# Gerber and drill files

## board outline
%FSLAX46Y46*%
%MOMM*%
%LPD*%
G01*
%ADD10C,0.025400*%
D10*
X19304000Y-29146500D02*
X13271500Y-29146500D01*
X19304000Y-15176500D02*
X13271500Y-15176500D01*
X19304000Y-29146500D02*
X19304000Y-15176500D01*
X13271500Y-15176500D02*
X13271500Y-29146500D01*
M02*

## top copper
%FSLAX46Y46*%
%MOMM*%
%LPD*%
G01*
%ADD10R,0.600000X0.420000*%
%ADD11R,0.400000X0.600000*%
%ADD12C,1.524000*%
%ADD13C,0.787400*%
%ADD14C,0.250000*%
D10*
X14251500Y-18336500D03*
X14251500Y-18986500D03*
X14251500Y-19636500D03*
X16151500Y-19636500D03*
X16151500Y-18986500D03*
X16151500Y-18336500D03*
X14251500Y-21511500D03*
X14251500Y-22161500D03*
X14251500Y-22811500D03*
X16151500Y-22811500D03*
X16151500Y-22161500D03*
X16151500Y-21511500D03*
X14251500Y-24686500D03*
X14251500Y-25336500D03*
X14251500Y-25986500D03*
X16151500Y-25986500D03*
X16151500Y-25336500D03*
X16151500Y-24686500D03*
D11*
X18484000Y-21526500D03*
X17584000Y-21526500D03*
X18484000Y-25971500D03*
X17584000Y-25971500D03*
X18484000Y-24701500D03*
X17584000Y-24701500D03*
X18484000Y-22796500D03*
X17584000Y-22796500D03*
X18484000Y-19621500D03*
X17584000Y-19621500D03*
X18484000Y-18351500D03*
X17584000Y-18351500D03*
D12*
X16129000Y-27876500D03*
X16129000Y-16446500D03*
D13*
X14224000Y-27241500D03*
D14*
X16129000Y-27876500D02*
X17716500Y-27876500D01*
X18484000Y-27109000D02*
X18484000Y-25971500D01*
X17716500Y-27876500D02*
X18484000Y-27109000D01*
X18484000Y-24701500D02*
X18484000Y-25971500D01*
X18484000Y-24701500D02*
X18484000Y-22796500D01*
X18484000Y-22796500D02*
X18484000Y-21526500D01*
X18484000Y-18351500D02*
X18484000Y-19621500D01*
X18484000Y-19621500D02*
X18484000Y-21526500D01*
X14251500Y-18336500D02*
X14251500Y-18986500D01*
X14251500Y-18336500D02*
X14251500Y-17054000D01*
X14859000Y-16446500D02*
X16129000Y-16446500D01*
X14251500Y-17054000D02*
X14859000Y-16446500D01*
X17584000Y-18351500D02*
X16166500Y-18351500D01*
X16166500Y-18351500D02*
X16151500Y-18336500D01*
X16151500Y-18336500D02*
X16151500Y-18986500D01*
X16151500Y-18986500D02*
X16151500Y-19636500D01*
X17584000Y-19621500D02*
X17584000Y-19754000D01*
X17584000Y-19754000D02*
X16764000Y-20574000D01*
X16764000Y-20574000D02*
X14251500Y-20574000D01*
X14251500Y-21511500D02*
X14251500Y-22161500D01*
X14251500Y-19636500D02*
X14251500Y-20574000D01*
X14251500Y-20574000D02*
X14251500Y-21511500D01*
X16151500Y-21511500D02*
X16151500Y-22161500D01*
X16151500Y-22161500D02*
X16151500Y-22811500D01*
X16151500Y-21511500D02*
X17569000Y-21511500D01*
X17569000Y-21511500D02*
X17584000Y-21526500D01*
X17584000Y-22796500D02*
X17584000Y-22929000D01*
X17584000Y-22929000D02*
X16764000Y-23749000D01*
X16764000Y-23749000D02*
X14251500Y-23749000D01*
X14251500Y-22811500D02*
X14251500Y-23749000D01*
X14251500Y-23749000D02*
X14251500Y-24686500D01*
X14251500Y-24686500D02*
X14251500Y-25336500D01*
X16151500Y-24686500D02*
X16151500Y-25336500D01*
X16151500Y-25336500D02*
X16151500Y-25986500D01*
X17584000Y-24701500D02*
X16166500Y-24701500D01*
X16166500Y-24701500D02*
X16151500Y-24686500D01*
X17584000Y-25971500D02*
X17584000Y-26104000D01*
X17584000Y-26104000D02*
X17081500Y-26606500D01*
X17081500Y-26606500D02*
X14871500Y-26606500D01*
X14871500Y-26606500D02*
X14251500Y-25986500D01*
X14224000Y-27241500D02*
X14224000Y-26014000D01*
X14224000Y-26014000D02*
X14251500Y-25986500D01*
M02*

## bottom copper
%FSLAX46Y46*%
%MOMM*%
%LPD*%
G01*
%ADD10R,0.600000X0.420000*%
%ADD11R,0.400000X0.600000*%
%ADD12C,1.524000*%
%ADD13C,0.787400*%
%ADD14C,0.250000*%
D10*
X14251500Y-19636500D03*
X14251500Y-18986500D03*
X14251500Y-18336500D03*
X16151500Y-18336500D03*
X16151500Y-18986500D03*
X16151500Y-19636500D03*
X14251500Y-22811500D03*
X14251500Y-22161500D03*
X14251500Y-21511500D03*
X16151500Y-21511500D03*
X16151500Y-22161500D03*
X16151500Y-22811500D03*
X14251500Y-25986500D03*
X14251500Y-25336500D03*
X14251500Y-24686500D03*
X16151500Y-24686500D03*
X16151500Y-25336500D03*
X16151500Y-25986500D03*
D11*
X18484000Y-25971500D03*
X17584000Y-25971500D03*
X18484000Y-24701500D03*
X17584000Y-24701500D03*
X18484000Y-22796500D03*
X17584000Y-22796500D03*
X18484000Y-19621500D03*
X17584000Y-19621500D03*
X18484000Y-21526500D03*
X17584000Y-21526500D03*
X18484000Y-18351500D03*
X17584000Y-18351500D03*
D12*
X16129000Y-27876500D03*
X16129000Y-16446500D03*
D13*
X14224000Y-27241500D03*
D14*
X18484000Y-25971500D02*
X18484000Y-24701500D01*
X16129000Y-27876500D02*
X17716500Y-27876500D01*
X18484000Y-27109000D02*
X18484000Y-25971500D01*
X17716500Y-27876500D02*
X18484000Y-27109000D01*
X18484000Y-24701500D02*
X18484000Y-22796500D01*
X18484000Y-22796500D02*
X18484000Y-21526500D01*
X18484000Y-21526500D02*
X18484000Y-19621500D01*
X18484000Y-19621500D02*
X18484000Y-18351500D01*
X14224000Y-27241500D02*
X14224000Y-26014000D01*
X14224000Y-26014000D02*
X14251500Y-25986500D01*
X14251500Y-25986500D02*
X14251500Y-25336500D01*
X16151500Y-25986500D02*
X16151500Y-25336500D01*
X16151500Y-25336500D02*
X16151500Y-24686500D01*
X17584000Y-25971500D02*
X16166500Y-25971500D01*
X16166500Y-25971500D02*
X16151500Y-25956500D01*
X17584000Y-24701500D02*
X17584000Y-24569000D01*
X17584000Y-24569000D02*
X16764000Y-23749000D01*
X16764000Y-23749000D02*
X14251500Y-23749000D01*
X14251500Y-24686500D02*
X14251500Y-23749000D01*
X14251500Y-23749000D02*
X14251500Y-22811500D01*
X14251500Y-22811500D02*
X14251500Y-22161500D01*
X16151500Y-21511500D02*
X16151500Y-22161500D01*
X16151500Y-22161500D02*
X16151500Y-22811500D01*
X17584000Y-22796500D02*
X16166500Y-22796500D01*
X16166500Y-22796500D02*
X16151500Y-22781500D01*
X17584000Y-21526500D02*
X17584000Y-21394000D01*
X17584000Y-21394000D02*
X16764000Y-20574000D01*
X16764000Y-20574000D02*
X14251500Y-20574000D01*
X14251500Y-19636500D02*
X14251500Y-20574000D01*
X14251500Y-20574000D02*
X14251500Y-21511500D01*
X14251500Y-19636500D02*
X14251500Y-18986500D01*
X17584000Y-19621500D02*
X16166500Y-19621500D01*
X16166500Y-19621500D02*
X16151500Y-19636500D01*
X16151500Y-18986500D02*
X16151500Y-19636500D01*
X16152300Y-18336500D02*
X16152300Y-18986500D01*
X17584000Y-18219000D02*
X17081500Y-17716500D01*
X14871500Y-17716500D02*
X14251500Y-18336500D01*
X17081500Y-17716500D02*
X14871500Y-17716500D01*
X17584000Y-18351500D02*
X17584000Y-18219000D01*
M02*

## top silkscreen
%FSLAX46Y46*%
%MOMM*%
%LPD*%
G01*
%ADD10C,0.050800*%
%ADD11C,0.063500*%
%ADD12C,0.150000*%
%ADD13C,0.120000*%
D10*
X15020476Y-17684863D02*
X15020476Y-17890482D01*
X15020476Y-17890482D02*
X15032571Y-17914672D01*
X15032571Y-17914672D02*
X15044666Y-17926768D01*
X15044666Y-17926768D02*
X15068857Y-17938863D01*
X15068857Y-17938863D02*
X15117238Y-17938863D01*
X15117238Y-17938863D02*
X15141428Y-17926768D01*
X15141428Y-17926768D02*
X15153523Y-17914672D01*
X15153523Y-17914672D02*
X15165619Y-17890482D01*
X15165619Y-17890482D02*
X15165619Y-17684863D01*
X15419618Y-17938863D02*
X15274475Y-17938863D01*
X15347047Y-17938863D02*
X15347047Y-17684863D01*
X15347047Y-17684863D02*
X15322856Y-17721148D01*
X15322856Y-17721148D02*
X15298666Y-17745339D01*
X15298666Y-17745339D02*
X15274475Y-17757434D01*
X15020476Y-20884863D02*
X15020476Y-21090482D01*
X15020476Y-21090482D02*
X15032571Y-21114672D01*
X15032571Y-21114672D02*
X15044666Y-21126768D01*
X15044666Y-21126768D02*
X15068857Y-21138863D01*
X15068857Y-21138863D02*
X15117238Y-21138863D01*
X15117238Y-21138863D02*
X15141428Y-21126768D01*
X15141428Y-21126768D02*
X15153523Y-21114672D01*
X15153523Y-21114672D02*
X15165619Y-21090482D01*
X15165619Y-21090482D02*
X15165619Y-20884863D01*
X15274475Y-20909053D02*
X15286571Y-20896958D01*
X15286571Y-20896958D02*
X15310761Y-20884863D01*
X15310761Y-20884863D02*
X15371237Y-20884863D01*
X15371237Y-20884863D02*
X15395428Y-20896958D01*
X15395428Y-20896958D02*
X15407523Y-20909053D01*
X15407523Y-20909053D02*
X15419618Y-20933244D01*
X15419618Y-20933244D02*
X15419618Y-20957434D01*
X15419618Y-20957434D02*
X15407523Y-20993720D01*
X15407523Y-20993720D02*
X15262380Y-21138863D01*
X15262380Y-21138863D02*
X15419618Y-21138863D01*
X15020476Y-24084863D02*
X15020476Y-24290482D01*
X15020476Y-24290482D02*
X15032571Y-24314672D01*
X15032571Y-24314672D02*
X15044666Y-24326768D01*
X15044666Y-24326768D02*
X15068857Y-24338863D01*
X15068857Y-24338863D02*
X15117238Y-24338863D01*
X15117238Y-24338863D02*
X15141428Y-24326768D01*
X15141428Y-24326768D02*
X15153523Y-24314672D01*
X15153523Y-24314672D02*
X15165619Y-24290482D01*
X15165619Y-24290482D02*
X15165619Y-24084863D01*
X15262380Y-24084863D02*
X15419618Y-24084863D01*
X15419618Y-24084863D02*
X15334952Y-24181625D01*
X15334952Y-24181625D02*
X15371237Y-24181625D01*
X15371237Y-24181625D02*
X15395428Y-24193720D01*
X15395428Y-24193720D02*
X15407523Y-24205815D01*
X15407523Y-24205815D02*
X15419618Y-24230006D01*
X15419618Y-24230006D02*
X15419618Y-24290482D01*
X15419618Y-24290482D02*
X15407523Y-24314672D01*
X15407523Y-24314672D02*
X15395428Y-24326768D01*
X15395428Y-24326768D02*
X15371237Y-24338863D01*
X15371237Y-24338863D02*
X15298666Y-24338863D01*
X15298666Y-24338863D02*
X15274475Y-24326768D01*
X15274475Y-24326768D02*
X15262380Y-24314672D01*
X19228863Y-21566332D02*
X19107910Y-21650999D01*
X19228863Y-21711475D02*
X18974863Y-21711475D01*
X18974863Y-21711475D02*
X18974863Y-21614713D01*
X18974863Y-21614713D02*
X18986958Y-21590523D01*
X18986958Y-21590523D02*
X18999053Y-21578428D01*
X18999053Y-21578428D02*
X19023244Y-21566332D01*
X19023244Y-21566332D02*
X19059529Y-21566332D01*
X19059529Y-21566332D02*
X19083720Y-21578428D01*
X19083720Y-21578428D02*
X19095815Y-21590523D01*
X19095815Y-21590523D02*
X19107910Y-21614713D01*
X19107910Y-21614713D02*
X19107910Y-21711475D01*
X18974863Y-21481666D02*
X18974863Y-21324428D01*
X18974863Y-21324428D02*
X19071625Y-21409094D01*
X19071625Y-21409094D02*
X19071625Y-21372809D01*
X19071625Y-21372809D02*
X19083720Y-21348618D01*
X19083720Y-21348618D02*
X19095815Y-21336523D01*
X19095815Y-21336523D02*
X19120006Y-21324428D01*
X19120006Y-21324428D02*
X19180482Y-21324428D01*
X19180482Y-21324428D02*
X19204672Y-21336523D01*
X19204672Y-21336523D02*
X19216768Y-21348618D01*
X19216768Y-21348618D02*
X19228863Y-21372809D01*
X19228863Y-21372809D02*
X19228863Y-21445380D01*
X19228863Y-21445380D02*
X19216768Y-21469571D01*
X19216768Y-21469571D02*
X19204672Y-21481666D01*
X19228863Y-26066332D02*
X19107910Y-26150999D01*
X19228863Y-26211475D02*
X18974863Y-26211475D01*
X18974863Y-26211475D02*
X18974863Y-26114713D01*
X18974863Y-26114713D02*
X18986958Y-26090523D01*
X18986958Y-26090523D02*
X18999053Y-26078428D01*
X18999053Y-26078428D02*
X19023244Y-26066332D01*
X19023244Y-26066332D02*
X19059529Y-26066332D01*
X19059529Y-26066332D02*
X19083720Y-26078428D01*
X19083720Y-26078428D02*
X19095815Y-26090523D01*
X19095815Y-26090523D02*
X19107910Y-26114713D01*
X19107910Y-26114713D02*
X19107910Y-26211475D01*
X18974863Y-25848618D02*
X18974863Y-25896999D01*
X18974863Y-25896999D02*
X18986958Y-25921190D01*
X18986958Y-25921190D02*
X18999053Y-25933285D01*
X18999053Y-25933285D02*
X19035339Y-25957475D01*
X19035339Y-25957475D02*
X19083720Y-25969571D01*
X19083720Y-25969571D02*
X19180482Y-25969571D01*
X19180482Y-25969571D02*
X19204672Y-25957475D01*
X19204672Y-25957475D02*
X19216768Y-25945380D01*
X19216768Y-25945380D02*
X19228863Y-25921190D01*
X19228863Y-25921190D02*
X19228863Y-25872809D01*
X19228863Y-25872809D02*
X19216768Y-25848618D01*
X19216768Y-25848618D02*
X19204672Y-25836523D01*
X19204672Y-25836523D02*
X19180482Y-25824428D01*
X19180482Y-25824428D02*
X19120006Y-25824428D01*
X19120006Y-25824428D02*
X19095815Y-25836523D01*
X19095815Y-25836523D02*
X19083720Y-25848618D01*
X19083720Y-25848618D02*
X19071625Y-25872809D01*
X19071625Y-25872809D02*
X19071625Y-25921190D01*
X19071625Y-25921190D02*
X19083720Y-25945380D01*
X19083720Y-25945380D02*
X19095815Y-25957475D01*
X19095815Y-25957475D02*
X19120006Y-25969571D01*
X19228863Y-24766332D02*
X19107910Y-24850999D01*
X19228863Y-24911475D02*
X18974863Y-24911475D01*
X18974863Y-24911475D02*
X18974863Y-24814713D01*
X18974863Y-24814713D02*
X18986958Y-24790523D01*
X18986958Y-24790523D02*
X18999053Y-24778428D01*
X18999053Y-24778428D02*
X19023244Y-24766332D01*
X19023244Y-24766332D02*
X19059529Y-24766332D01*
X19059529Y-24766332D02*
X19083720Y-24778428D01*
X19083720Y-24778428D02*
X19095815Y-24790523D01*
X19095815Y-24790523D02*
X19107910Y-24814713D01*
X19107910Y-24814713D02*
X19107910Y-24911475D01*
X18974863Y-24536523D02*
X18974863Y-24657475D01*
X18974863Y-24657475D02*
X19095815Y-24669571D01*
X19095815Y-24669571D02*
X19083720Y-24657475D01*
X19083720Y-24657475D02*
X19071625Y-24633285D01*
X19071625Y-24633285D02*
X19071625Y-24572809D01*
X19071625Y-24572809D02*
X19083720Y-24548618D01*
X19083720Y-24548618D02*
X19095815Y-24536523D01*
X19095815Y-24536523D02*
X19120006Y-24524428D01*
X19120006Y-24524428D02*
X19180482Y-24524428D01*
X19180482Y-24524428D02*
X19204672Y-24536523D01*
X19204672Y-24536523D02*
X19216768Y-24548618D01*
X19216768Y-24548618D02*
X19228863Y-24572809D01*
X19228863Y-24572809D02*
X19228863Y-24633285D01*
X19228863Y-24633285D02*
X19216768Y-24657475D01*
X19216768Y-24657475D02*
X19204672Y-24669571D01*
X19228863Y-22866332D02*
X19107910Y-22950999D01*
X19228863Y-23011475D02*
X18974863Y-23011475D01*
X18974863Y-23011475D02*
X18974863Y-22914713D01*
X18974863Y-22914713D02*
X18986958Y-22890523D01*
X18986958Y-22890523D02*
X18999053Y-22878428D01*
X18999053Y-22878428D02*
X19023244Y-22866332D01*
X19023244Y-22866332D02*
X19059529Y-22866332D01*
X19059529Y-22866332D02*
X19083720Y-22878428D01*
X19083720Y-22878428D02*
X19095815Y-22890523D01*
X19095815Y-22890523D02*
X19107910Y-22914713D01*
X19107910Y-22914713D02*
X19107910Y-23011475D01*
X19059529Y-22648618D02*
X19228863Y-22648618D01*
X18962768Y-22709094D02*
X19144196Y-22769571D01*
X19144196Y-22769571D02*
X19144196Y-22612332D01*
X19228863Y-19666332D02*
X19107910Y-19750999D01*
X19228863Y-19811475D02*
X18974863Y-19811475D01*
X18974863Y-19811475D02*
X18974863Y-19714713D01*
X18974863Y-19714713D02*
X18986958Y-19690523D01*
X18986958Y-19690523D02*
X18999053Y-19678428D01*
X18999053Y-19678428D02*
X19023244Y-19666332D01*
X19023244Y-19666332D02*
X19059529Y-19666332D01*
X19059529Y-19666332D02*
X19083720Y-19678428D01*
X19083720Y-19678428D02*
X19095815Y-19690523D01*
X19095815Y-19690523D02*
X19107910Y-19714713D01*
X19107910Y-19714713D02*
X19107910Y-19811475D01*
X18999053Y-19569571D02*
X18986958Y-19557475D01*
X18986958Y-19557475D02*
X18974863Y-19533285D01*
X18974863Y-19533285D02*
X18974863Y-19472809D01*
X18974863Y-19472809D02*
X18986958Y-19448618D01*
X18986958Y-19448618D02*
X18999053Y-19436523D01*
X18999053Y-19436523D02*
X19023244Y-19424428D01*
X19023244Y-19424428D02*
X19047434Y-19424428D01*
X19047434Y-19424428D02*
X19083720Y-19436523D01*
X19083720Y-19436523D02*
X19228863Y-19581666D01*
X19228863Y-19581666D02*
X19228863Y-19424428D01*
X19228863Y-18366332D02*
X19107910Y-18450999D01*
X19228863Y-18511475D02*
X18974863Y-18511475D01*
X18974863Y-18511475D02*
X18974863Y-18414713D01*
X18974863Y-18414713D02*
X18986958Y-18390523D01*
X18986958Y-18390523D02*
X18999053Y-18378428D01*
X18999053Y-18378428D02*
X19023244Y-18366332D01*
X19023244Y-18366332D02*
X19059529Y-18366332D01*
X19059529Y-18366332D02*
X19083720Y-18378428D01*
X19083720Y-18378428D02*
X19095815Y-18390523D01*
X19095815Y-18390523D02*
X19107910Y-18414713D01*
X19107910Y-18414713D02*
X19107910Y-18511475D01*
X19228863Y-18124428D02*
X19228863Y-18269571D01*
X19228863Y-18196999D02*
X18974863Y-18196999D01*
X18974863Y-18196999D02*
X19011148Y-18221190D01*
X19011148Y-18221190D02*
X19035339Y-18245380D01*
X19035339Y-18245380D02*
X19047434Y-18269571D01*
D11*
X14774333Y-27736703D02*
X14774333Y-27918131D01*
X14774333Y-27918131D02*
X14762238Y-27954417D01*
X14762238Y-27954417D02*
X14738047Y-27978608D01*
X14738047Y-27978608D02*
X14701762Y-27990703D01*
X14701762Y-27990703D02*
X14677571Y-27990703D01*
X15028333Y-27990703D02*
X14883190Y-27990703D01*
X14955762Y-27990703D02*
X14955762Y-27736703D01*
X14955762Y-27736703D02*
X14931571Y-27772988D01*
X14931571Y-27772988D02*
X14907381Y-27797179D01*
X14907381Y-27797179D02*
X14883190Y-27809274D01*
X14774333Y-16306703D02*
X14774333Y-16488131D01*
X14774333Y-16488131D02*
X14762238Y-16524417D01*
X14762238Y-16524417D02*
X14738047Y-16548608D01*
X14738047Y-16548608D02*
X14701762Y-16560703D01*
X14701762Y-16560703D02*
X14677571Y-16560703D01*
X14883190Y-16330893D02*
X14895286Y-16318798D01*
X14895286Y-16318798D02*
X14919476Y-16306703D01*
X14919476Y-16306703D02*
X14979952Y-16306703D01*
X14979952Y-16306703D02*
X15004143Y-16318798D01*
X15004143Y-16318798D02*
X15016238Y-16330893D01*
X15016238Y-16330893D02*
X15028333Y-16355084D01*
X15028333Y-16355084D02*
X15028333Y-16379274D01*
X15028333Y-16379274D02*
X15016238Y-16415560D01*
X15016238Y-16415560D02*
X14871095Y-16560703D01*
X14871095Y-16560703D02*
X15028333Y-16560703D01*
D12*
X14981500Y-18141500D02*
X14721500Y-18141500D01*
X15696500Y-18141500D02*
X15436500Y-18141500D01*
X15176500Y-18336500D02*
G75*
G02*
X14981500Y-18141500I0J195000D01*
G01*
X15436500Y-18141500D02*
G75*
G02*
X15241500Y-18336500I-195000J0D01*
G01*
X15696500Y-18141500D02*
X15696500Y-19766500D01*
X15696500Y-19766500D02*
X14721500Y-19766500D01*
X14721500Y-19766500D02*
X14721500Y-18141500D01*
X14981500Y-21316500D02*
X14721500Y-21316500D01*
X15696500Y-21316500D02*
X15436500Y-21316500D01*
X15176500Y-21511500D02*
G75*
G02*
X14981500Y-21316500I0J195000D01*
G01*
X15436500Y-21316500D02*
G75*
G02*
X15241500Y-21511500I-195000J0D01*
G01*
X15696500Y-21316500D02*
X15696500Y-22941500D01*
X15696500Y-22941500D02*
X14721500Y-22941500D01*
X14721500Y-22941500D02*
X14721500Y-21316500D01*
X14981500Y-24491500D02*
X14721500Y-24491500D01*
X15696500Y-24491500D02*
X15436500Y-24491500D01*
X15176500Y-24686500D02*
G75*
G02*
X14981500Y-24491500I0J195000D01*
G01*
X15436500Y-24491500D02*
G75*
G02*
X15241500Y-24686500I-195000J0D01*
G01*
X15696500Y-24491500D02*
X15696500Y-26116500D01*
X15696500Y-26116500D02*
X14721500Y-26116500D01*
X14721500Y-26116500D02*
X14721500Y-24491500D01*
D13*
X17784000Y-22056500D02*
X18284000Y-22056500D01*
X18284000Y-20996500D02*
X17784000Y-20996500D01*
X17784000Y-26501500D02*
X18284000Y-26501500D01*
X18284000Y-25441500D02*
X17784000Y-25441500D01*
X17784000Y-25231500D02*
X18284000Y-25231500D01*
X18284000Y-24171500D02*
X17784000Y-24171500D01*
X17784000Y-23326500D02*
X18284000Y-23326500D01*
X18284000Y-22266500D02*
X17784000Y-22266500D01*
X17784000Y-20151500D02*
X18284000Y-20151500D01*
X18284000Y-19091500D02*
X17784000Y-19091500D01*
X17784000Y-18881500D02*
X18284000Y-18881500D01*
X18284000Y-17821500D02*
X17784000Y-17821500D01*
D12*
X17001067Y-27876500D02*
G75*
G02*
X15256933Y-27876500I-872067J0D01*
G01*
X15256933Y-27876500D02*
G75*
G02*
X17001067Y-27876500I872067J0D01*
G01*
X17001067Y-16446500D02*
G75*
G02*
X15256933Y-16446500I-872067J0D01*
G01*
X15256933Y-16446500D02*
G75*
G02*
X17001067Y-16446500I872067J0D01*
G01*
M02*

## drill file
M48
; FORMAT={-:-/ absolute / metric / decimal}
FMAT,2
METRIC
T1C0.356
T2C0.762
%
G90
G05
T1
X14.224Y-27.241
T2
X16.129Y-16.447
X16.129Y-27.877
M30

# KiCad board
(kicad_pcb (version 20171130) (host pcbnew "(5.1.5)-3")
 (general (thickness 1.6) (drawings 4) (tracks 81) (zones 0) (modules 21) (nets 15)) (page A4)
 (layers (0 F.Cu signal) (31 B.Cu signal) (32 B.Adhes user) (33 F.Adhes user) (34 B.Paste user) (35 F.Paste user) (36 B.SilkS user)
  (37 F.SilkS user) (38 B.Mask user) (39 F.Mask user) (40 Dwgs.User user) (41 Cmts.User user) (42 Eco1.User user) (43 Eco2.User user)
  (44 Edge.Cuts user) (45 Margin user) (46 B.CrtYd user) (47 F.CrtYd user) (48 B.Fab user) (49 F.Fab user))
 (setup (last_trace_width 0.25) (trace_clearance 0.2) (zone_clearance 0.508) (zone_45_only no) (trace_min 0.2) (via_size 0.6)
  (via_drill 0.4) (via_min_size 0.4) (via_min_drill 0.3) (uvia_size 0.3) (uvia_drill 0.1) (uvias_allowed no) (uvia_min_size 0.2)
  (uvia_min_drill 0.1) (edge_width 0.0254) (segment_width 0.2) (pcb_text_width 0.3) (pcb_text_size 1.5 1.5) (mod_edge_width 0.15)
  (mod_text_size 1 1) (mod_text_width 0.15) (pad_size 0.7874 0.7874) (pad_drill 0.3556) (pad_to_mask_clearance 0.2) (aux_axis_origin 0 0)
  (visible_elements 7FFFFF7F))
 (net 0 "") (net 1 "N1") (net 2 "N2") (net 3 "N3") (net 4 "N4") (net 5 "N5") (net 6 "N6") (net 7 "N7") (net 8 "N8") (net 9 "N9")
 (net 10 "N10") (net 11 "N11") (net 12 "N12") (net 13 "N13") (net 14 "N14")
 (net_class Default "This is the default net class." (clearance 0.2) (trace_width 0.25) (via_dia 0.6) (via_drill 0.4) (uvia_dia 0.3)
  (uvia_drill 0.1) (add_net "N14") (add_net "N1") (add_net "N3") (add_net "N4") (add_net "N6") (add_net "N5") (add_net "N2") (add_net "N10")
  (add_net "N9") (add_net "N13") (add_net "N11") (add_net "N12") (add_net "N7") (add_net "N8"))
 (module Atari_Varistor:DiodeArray (layer F.Cu) (at 15.1765 18.9865 270)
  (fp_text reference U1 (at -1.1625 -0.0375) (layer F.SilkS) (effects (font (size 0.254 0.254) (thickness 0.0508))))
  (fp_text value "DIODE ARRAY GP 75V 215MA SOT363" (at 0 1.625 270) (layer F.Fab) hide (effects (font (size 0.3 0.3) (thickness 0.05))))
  (fp_line (start -0.845 0.195) (end -0.845 0.455) (layer F.SilkS) (width 0.15))
  (fp_line (start -0.845 -0.52) (end -0.845 -0.26) (layer F.SilkS) (width 0.15))
  (fp_arc (start -0.845 0) (end -0.65 0) (angle 90) (layer F.SilkS) (width 0.15))
  (fp_arc (start -0.845 -0.065) (end -0.845 -0.26) (angle 90) (layer F.SilkS) (width 0.15))
  (fp_line (start -0.845 -0.52) (end 0.78 -0.52) (layer F.SilkS) (width 0.15))
  (fp_line (start 0.78 -0.52) (end 0.78 0.455) (layer F.SilkS) (width 0.15))
  (fp_line (start 0.78 0.455) (end -0.845 0.455) (layer F.SilkS) (width 0.15))
  (pad 1 smd rect (at -0.65 0.925 270) (size 0.42 0.6) (layers F.Cu F.Paste F.Mask) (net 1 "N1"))
  (pad 2 smd rect (at 0 0.925 270) (size 0.42 0.6) (layers F.Cu F.Paste F.Mask) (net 1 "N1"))
  (pad 3 smd rect (at 0.65 0.925 270) (size 0.42 0.6) (layers F.Cu F.Paste F.Mask) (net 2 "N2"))
  (pad 4 smd rect (at 0.65 -0.975 270) (size 0.42 0.6) (layers F.Cu F.Paste F.Mask) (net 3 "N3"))
  (pad 5 smd rect (at 0 -0.975 270) (size 0.42 0.6) (layers F.Cu F.Paste F.Mask) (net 3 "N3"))
  (pad 6 smd rect (at -0.65 -0.975 270) (size 0.42 0.6) (layers F.Cu F.Paste F.Mask) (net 3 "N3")))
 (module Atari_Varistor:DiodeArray (layer B.Cu) (at 15.1765 18.9865 90)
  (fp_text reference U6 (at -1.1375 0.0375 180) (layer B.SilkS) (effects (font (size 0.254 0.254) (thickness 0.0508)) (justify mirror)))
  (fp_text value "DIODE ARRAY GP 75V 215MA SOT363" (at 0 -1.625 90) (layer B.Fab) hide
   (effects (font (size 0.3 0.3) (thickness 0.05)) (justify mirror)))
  (pad 1 smd rect (at -0.65 -0.925 90) (size 0.42 0.6) (layers B.Cu B.Paste B.Mask) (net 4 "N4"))
  (pad 2 smd rect (at 0 -0.925 90) (size 0.42 0.6) (layers B.Cu B.Paste B.Mask) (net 4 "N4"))
  (pad 3 smd rect (at 0.65 -0.925 90) (size 0.42 0.6) (layers B.Cu B.Paste B.Mask) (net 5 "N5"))
  (pad 4 smd rect (at 0.65 0.975 90) (size 0.42 0.6) (layers B.Cu B.Paste B.Mask) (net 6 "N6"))
  (pad 5 smd rect (at 0 0.975 90) (size 0.42 0.6) (layers B.Cu B.Paste B.Mask) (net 6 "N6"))
  (pad 6 smd rect (at -0.65 0.975 90) (size 0.42 0.6) (layers B.Cu B.Paste B.Mask) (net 6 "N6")))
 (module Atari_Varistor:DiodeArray (layer B.Cu) (at 15.1765 22.1615 90)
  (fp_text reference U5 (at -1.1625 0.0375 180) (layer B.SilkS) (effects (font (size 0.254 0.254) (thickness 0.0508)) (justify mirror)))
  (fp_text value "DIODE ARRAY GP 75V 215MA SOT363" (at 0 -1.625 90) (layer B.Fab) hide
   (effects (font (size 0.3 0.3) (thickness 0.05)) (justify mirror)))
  (pad 1 smd rect (at -0.65 -0.925 90) (size 0.42 0.6) (layers B.Cu B.Paste B.Mask) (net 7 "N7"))
  (pad 2 smd rect (at 0 -0.925 90) (size 0.42 0.6) (layers B.Cu B.Paste B.Mask) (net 7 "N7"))
  (pad 3 smd rect (at 0.65 -0.925 90) (size 0.42 0.6) (layers B.Cu B.Paste B.Mask) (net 4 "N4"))
  (pad 4 smd rect (at 0.65 0.975 90) (size 0.42 0.6) (layers B.Cu B.Paste B.Mask) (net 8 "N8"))
  (pad 5 smd rect (at 0 0.975 90) (size 0.42 0.6) (layers B.Cu B.Paste B.Mask) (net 8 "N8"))
  (pad 6 smd rect (at -0.65 0.975 90) (size 0.42 0.6) (layers B.Cu B.Paste B.Mask) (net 8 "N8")))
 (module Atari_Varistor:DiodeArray (layer F.Cu) (at 15.1765 22.1615 270)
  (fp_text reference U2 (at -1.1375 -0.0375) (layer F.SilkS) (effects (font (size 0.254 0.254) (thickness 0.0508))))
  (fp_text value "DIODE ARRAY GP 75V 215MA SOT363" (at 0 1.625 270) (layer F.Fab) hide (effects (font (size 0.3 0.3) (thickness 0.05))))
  (fp_line (start -0.845 0.195) (end -0.845 0.455) (layer F.SilkS) (width 0.15))
  (fp_line (start -0.845 -0.52) (end -0.845 -0.26) (layer F.SilkS) (width 0.15))
  (fp_arc (start -0.845 0) (end -0.65 0) (angle 90) (layer F.SilkS) (width 0.15))
  (fp_arc (start -0.845 -0.065) (end -0.845 -0.26) (angle 90) (layer F.SilkS) (width 0.15))
  (fp_line (start -0.845 -0.52) (end 0.78 -0.52) (layer F.SilkS) (width 0.15))
  (fp_line (start 0.78 -0.52) (end 0.78 0.455) (layer F.SilkS) (width 0.15))
  (fp_line (start 0.78 0.455) (end -0.845 0.455) (layer F.SilkS) (width 0.15))
  (pad 1 smd rect (at -0.65 0.925 270) (size 0.42 0.6) (layers F.Cu F.Paste F.Mask) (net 2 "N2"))
  (pad 2 smd rect (at 0 0.925 270) (size 0.42 0.6) (layers F.Cu F.Paste F.Mask) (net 2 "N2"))
  (pad 3 smd rect (at 0.65 0.925 270) (size 0.42 0.6) (layers F.Cu F.Paste F.Mask) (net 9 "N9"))
  (pad 4 smd rect (at 0.65 -0.975 270) (size 0.42 0.6) (layers F.Cu F.Paste F.Mask) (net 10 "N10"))
  (pad 5 smd rect (at 0 -0.975 270) (size 0.42 0.6) (layers F.Cu F.Paste F.Mask) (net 10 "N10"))
  (pad 6 smd rect (at -0.65 -0.975 270) (size 0.42 0.6) (layers F.Cu F.Paste F.Mask) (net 10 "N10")))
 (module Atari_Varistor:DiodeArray (layer B.Cu) (at 15.1765 25.3365 90)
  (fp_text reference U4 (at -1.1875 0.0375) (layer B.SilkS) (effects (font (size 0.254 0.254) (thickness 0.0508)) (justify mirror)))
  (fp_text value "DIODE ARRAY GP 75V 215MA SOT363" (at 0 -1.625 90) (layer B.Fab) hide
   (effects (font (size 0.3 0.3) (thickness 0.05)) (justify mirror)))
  (pad 1 smd rect (at -0.65 -0.925 90) (size 0.42 0.6) (layers B.Cu B.Paste B.Mask) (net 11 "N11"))
  (pad 2 smd rect (at 0 -0.925 90) (size 0.42 0.6) (layers B.Cu B.Paste B.Mask) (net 11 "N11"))
  (pad 3 smd rect (at 0.65 -0.925 90) (size 0.42 0.6) (layers B.Cu B.Paste B.Mask) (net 7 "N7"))
  (pad 4 smd rect (at 0.65 0.975 90) (size 0.42 0.6) (layers B.Cu B.Paste B.Mask) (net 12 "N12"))
  (pad 5 smd rect (at 0 0.975 90) (size 0.42 0.6) (layers B.Cu B.Paste B.Mask) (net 12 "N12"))
  (pad 6 smd rect (at -0.65 0.975 90) (size 0.42 0.6) (layers B.Cu B.Paste B.Mask) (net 12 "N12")))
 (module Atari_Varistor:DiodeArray (layer F.Cu) (at 15.1765 25.3365 270)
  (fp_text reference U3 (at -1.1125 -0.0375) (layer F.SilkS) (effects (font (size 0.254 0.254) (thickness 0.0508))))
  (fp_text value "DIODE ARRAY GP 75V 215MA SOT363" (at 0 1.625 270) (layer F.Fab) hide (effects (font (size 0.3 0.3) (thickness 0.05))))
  (fp_line (start -0.845 0.195) (end -0.845 0.455) (layer F.SilkS) (width 0.15))
  (fp_line (start -0.845 -0.52) (end -0.845 -0.26) (layer F.SilkS) (width 0.15))
  (fp_arc (start -0.845 0) (end -0.65 0) (angle 90) (layer F.SilkS) (width 0.15))
  (fp_arc (start -0.845 -0.065) (end -0.845 -0.26) (angle 90) (layer F.SilkS) (width 0.15))
  (fp_line (start -0.845 -0.52) (end 0.78 -0.52) (layer F.SilkS) (width 0.15))
  (fp_line (start 0.78 -0.52) (end 0.78 0.455) (layer F.SilkS) (width 0.15))
  (fp_line (start 0.78 0.455) (end -0.845 0.455) (layer F.SilkS) (width 0.15))
  (pad 1 smd rect (at -0.65 0.925 270) (size 0.42 0.6) (layers F.Cu F.Paste F.Mask) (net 9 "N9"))
  (pad 2 smd rect (at 0 0.925 270) (size 0.42 0.6) (layers F.Cu F.Paste F.Mask) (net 9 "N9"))
  (pad 3 smd rect (at 0.65 0.925 270) (size 0.42 0.6) (layers F.Cu F.Paste F.Mask) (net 11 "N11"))
  (pad 4 smd rect (at 0.65 -0.975 270) (size 0.42 0.6) (layers F.Cu F.Paste F.Mask) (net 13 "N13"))
  (pad 5 smd rect (at 0 -0.975 270) (size 0.42 0.6) (layers F.Cu F.Paste F.Mask) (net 13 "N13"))
  (pad 6 smd rect (at -0.65 -0.975 270) (size 0.42 0.6) (layers F.Cu F.Paste F.Mask) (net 13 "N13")))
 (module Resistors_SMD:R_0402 (layer F.Cu) (at 18.034 21.5265 180)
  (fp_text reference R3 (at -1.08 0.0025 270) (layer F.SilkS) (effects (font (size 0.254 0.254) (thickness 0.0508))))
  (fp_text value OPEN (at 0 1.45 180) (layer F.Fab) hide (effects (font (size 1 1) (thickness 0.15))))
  (fp_line (start 0.25 -0.53) (end -0.25 -0.53) (layer F.SilkS) (width 0.12))
  (fp_line (start -0.25 0.53) (end 0.25 0.53) (layer F.SilkS) (width 0.12))
  (pad 1 smd rect (at -0.45 0 180) (size 0.4 0.6) (layers F.Cu F.Paste F.Mask) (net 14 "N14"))
  (pad 2 smd rect (at 0.45 0 180) (size 0.4 0.6) (layers F.Cu F.Paste F.Mask) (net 10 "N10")))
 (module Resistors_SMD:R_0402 (layer B.Cu) (at 18.034 25.9715 180)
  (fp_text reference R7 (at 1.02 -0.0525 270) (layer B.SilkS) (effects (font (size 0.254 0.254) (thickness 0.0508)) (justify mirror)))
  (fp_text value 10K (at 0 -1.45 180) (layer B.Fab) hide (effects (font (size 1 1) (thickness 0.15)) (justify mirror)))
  (pad 1 smd rect (at -0.45 0 180) (size 0.4 0.6) (layers B.Cu B.Paste B.Mask) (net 14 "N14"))
  (pad 2 smd rect (at 0.45 0 180) (size 0.4 0.6) (layers B.Cu B.Paste B.Mask) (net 12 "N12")))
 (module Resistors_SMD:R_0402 (layer B.Cu) (at 18.034 24.7015 180)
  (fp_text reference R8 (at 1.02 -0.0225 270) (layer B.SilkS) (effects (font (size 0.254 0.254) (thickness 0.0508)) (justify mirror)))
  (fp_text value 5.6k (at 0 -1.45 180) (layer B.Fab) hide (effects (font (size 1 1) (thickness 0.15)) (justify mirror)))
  (pad 1 smd rect (at -0.45 0 180) (size 0.4 0.6) (layers B.Cu B.Paste B.Mask) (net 14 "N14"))
  (pad 2 smd rect (at 0.45 0 180) (size 0.4 0.6) (layers B.Cu B.Paste B.Mask) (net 7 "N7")))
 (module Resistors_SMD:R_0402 (layer B.Cu) (at 18.034 22.7965 180)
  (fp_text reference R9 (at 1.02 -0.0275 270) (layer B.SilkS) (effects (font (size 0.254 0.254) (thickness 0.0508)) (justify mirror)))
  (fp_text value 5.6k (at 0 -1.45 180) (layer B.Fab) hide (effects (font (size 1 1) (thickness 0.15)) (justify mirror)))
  (pad 1 smd rect (at -0.45 0 180) (size 0.4 0.6) (layers B.Cu B.Paste B.Mask) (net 14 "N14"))
  (pad 2 smd rect (at 0.45 0 180) (size 0.4 0.6) (layers B.Cu B.Paste B.Mask) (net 8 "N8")))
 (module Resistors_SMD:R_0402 (layer B.Cu) (at 18.034 19.6215 180)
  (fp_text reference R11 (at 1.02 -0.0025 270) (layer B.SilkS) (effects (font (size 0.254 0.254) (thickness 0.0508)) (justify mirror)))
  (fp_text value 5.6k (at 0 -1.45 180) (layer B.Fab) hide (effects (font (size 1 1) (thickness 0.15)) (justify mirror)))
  (pad 1 smd rect (at -0.45 0 180) (size 0.4 0.6) (layers B.Cu B.Paste B.Mask) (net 14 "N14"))
  (pad 2 smd rect (at 0.45 0 180) (size 0.4 0.6) (layers B.Cu B.Paste B.Mask) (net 6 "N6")))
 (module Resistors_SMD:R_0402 (layer B.Cu) (at 18.034 21.5265 180)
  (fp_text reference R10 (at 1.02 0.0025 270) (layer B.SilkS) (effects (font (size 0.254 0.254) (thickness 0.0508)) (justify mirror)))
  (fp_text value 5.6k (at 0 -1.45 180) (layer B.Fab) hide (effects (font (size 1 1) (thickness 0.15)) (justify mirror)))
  (pad 1 smd rect (at -0.45 0 180) (size 0.4 0.6) (layers B.Cu B.Paste B.Mask) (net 14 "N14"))
  (pad 2 smd rect (at 0.45 0 180) (size 0.4 0.6) (layers B.Cu B.Paste B.Mask) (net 4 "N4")))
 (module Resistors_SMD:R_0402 (layer F.Cu) (at 18.034 25.9715 180)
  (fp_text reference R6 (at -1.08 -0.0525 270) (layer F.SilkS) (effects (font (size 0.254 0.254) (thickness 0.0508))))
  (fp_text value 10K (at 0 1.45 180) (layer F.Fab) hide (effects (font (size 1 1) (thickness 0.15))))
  (fp_line (start 0.25 -0.53) (end -0.25 -0.53) (layer F.SilkS) (width 0.12))
  (fp_line (start -0.25 0.53) (end 0.25 0.53) (layer F.SilkS) (width 0.12))
  (pad 1 smd rect (at -0.45 0 180) (size 0.4 0.6) (layers F.Cu F.Paste F.Mask) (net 14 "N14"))
  (pad 2 smd rect (at 0.45 0 180) (size 0.4 0.6) (layers F.Cu F.Paste F.Mask) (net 11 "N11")))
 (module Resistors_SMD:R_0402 (layer F.Cu) (at 18.034 24.7015 180)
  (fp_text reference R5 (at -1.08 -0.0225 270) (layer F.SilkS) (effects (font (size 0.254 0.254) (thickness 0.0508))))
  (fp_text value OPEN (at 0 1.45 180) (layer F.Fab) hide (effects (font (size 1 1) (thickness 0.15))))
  (fp_line (start 0.25 -0.53) (end -0.25 -0.53) (layer F.SilkS) (width 0.12))
  (fp_line (start -0.25 0.53) (end 0.25 0.53) (layer F.SilkS) (width 0.12))
  (pad 1 smd rect (at -0.45 0 180) (size 0.4 0.6) (layers F.Cu F.Paste F.Mask) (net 14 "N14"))
  (pad 2 smd rect (at 0.45 0 180) (size 0.4 0.6) (layers F.Cu F.Paste F.Mask) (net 13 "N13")))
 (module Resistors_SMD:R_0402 (layer F.Cu) (at 18.034 22.7965 180)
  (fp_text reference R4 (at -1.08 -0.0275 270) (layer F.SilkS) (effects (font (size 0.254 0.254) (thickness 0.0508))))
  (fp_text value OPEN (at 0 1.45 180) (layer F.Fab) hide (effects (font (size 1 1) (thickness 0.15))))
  (fp_line (start 0.25 -0.53) (end -0.25 -0.53) (layer F.SilkS) (width 0.12))
  (fp_line (start -0.25 0.53) (end 0.25 0.53) (layer F.SilkS) (width 0.12))
  (pad 1 smd rect (at -0.45 0 180) (size 0.4 0.6) (layers F.Cu F.Paste F.Mask) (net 14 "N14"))
  (pad 2 smd rect (at 0.45 0 180) (size 0.4 0.6) (layers F.Cu F.Paste F.Mask) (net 9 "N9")))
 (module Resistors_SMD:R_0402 (layer B.Cu) (at 18.034 18.3515 180)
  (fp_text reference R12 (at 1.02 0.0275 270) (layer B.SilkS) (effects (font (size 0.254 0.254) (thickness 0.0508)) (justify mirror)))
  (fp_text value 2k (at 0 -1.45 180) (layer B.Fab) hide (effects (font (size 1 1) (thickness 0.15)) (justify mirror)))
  (pad 1 smd rect (at -0.45 0 180) (size 0.4 0.6) (layers B.Cu B.Paste B.Mask) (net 14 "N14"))
  (pad 2 smd rect (at 0.45 0 180) (size 0.4 0.6) (layers B.Cu B.Paste B.Mask) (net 5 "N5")))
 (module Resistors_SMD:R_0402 (layer F.Cu) (at 18.034 19.6215 180)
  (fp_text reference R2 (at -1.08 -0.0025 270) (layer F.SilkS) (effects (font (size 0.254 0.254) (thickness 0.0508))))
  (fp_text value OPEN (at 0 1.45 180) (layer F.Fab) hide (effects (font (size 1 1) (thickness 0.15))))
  (fp_line (start 0.25 -0.53) (end -0.25 -0.53) (layer F.SilkS) (width 0.12))
  (fp_line (start -0.25 0.53) (end 0.25 0.53) (layer F.SilkS) (width 0.12))
  (pad 1 smd rect (at -0.45 0 180) (size 0.4 0.6) (layers F.Cu F.Paste F.Mask) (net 14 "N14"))
  (pad 2 smd rect (at 0.45 0 180) (size 0.4 0.6) (layers F.Cu F.Paste F.Mask) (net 2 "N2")))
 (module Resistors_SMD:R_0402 (layer F.Cu) (at 18.034 18.3515 180)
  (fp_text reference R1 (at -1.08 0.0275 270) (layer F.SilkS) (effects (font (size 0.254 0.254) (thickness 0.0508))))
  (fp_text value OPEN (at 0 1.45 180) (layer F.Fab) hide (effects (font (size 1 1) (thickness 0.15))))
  (fp_line (start 0.25 -0.53) (end -0.25 -0.53) (layer F.SilkS) (width 0.12))
  (fp_line (start -0.25 0.53) (end 0.25 0.53) (layer F.SilkS) (width 0.12))
  (pad 1 smd rect (at -0.45 0 180) (size 0.4 0.6) (layers F.Cu F.Paste F.Mask) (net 14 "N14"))
  (pad 2 smd rect (at 0.45 0 180) (size 0.4 0.6) (layers F.Cu F.Paste F.Mask) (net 3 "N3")))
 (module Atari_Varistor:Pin (layer F.Cu) (at 16.129 27.8765)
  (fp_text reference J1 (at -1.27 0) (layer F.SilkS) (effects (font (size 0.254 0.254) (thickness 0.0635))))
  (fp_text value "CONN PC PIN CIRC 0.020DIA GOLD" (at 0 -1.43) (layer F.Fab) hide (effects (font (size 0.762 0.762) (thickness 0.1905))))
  (fp_circle (center 0 0) (end 0.78 0.39) (layer F.SilkS) (width 0.15))
  (pad 1 thru_hole circle (at 0 0) (size 1.524 1.524) (drill 0.762) (layers *.Cu *.Mask) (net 14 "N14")))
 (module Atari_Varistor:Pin (layer F.Cu) (at 16.129 16.4465)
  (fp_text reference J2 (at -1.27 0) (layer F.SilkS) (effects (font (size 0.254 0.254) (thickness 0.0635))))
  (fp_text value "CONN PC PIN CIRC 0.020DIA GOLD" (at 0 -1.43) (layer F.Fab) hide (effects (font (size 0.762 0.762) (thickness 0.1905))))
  (fp_circle (center 0 0) (end 0.78 0.39) (layer F.SilkS) (width 0.15))
  (pad 1 thru_hole circle (at 0 0) (size 1.524 1.524) (drill 0.762) (layers *.Cu *.Mask) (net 1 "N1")))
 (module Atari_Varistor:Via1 (layer F.Cu) (at 14.224 27.2415)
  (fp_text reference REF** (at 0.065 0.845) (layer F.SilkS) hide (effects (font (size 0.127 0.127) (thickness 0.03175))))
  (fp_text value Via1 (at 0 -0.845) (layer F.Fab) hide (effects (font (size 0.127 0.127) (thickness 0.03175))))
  (pad 1 thru_hole circle (at 0 0) (size 0.7874 0.7874) (drill 0.3556) (layers *.Cu *.Mask) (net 11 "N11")))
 (gr_line (start 19.304 29.1465) (end 13.2715 29.1465) (angle 90) (layer Edge.Cuts) (width 0.0254))
 (gr_line (start 19.304 15.1765) (end 13.2715 15.1765) (angle 90) (layer Edge.Cuts) (width 0.0254))
 (gr_line (start 19.304 29.1465) (end 19.304 15.1765) (angle 90) (layer Edge.Cuts) (width 0.0254))
 (gr_line (start 13.2715 15.1765) (end 13.2715 29.1465) (angle 90) (layer Edge.Cuts) (width 0.0254))
 (segment (start 18.484 25.9715) (end 18.484 24.7015) (width 0.25) (layer B.Cu) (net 14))
 (segment (start 16.129 27.8765) (end 17.7165 27.8765) (width 0.25) (layer B.Cu) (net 14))
 (segment (start 18.484 27.109) (end 18.484 25.9715) (width 0.25) (layer B.Cu) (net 14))
 (segment (start 17.7165 27.8765) (end 18.484 27.109) (width 0.25) (layer B.Cu) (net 14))
 (segment (start 16.129 27.8765) (end 17.7165 27.8765) (width 0.25) (layer F.Cu) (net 14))
 (segment (start 18.484 27.109) (end 18.484 25.9715) (width 0.25) (layer F.Cu) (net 14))
 (segment (start 17.7165 27.8765) (end 18.484 27.109) (width 0.25) (layer F.Cu) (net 14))
 (segment (start 18.484 24.7015) (end 18.484 25.9715) (width 0.25) (layer F.Cu) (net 14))
 (segment (start 18.484 24.7015) (end 18.484 22.7965) (width 0.25) (layer B.Cu) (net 14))
 (segment (start 18.484 22.7965) (end 18.484 21.5265) (width 0.25) (layer B.Cu) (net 14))
 (segment (start 18.484 21.5265) (end 18.484 19.6215) (width 0.25) (layer B.Cu) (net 14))
 (segment (start 18.484 19.6215) (end 18.484 18.3515) (width 0.25) (layer B.Cu) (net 14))
 (segment (start 18.484 24.7015) (end 18.484 22.7965) (width 0.25) (layer F.Cu) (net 14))
 (segment (start 18.484 22.7965) (end 18.484 21.5265) (width 0.25) (layer F.Cu) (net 14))
 (segment (start 18.484 18.3515) (end 18.484 19.6215) (width 0.25) (layer F.Cu) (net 14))
 (segment (start 18.484 19.6215) (end 18.484 21.5265) (width 0.25) (layer F.Cu) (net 14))
 (segment (start 14.2515 18.3365) (end 14.2515 18.9865) (width 0.25) (layer F.Cu) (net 1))
 (segment (start 14.2515 18.3365) (end 14.2515 17.054) (width 0.25) (layer F.Cu) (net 1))
 (segment (start 14.859 16.4465) (end 16.129 16.4465) (width 0.25) (layer F.Cu) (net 1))
 (segment (start 14.2515 17.054) (end 14.859 16.4465) (width 0.25) (layer F.Cu) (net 1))
 (segment (start 17.584 18.3515) (end 16.1665 18.3515) (width 0.25) (layer F.Cu) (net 3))
 (segment (start 16.1665 18.3515) (end 16.1515 18.3365) (width 0.25) (layer F.Cu) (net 3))
 (segment (start 16.1515 18.3365) (end 16.1515 18.9865) (width 0.25) (layer F.Cu) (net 3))
 (segment (start 16.1515 18.9865) (end 16.1515 19.6365) (width 0.25) (layer F.Cu) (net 3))
 (segment (start 17.584 19.6215) (end 17.584 19.754) (width 0.25) (layer F.Cu) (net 2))
 (segment (start 17.584 19.754) (end 16.764 20.574) (width 0.25) (layer F.Cu) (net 2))
 (segment (start 16.764 20.574) (end 14.2515 20.574) (width 0.25) (layer F.Cu) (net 2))
 (segment (start 14.2515 21.5115) (end 14.2515 22.1615) (width 0.25) (layer F.Cu) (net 2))
 (segment (start 14.2515 19.6365) (end 14.2515 20.574) (width 0.25) (layer F.Cu) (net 2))
 (segment (start 14.2515 20.574) (end 14.2515 21.5115) (width 0.25) (layer F.Cu) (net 2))
 (segment (start 16.1515 21.5115) (end 16.1515 22.1615) (width 0.25) (layer F.Cu) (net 10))
 (segment (start 16.1515 22.1615) (end 16.1515 22.8115) (width 0.25) (layer F.Cu) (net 10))
 (segment (start 16.1515 21.5115) (end 17.569 21.5115) (width 0.25) (layer F.Cu) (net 10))
 (segment (start 17.569 21.5115) (end 17.584 21.5265) (width 0.25) (layer F.Cu) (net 10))
 (segment (start 17.584 22.7965) (end 17.584 22.929) (width 0.25) (layer F.Cu) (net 9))
 (segment (start 17.584 22.929) (end 16.764 23.749) (width 0.25) (layer F.Cu) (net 9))
 (segment (start 16.764 23.749) (end 14.2515 23.749) (width 0.25) (layer F.Cu) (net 9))
 (segment (start 14.2515 22.8115) (end 14.2515 23.749) (width 0.25) (layer F.Cu) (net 9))
 (segment (start 14.2515 23.749) (end 14.2515 24.6865) (width 0.25) (layer F.Cu) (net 9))
 (segment (start 14.2515 24.6865) (end 14.2515 25.3365) (width 0.25) (layer F.Cu) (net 9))
 (segment (start 16.1515 24.6865) (end 16.1515 25.3365) (width 0.25) (layer F.Cu) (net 13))
 (segment (start 16.1515 25.3365) (end 16.1515 25.9865) (width 0.25) (layer F.Cu) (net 13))
 (segment (start 17.584 24.7015) (end 16.1665 24.7015) (width 0.25) (layer F.Cu) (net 13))
 (segment (start 16.1665 24.7015) (end 16.1515 24.6865) (width 0.25) (layer F.Cu) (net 13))
 (segment (start 17.584 25.9715) (end 17.584 26.104) (width 0.25) (layer F.Cu) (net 11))
 (segment (start 17.584 26.104) (end 17.0815 26.6065) (width 0.25) (layer F.Cu) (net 11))
 (segment (start 17.0815 26.6065) (end 14.8715 26.6065) (width 0.25) (layer F.Cu) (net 11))
 (segment (start 14.8715 26.6065) (end 14.2515 25.9865) (width 0.25) (layer F.Cu) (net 11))
 (segment (start 14.224 27.2415) (end 14.224 26.014) (width 0.25) (layer B.Cu) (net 11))
 (segment (start 14.224 26.014) (end 14.2515 25.9865) (width 0.25) (layer B.Cu) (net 11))
 (segment (start 14.224 27.2415) (end 14.224 26.014) (width 0.25) (layer F.Cu) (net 11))
 (segment (start 14.224 26.014) (end 14.2515 25.9865) (width 0.25) (layer F.Cu) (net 11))
 (segment (start 14.2515 25.9865) (end 14.2515 25.3365) (width 0.25) (layer B.Cu) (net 11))
 (segment (start 16.1515 25.9865) (end 16.1515 25.3365) (width 0.25) (layer B.Cu) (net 12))
 (segment (start 16.1515 25.3365) (end 16.1515 24.6865) (width 0.25) (layer B.Cu) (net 12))
 (segment (start 17.584 25.9715) (end 16.1665 25.9715) (width 0.25) (layer B.Cu) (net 12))
 (segment (start 16.1665 25.9715) (end 16.1515 25.9565) (width 0.25) (layer B.Cu) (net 12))
 (segment (start 17.584 24.7015) (end 17.584 24.569) (width 0.25) (layer B.Cu) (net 7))
 (segment (start 17.584 24.569) (end 16.764 23.749) (width 0.25) (layer B.Cu) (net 7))
 (segment (start 16.764 23.749) (end 14.2515 23.749) (width 0.25) (layer B.Cu) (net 7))
 (segment (start 14.2515 24.6865) (end 14.2515 23.749) (width 0.25) (layer B.Cu) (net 7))
 (segment (start 14.2515 23.749) (end 14.2515 22.8115) (width 0.25) (layer B.Cu) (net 7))
 (segment (start 14.2515 22.8115) (end 14.2515 22.1615) (width 0.25) (layer B.Cu) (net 7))
 (segment (start 16.1515 21.5115) (end 16.1515 22.1615) (width 0.25) (layer B.Cu) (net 8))
 (segment (start 16.1515 22.1615) (end 16.1515 22.8115) (width 0.25) (layer B.Cu) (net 8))
 (segment (start 17.584 22.7965) (end 16.1665 22.7965) (width 0.25) (layer B.Cu) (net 8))
 (segment (start 16.1665 22.7965) (end 16.1515 22.7815) (width 0.25) (layer B.Cu) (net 8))
 (segment (start 17.584 21.5265) (end 17.584 21.394) (width 0.25) (layer B.Cu) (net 4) (status C00000))
 (segment (start 17.584 21.394) (end 16.764 20.574) (width 0.25) (layer B.Cu) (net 4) (status 400000))
 (segment (start 16.764 20.574) (end 14.2515 20.574) (width 0.25) (layer B.Cu) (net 4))
 (segment (start 14.2515 19.6365) (end 14.2515 20.574) (width 0.25) (layer B.Cu) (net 4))
 (segment (start 14.2515 20.574) (end 14.2515 21.5115) (width 0.25) (layer B.Cu) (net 4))
 (segment (start 14.2515 19.6365) (end 14.2515 18.9865) (width 0.25) (layer B.Cu) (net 4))
 (segment (start 17.584 19.6215) (end 16.1665 19.6215) (width 0.25) (layer B.Cu) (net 6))
 (segment (start 16.1665 19.6215) (end 16.1515 19.6365) (width 0.25) (layer B.Cu) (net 6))
 (segment (start 16.1515 18.9865) (end 16.1515 19.6365) (width 0.25) (layer B.Cu) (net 6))
 (segment (start 16.1523 18.3365) (end 16.1523 18.9865) (width 0.25) (layer B.Cu) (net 6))
 (segment (start 17.584 18.219) (end 17.0815 17.7165) (width 0.25) (layer B.Cu) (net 5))
 (segment (start 14.8715 17.7165) (end 14.2515 18.3365) (width 0.25) (layer B.Cu) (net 5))
 (segment (start 17.0815 17.7165) (end 14.8715 17.7165) (width 0.25) (layer B.Cu) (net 5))
 (segment (start 17.584 18.3515) (end 17.584 18.219) (width 0.25) (layer B.Cu) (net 5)))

